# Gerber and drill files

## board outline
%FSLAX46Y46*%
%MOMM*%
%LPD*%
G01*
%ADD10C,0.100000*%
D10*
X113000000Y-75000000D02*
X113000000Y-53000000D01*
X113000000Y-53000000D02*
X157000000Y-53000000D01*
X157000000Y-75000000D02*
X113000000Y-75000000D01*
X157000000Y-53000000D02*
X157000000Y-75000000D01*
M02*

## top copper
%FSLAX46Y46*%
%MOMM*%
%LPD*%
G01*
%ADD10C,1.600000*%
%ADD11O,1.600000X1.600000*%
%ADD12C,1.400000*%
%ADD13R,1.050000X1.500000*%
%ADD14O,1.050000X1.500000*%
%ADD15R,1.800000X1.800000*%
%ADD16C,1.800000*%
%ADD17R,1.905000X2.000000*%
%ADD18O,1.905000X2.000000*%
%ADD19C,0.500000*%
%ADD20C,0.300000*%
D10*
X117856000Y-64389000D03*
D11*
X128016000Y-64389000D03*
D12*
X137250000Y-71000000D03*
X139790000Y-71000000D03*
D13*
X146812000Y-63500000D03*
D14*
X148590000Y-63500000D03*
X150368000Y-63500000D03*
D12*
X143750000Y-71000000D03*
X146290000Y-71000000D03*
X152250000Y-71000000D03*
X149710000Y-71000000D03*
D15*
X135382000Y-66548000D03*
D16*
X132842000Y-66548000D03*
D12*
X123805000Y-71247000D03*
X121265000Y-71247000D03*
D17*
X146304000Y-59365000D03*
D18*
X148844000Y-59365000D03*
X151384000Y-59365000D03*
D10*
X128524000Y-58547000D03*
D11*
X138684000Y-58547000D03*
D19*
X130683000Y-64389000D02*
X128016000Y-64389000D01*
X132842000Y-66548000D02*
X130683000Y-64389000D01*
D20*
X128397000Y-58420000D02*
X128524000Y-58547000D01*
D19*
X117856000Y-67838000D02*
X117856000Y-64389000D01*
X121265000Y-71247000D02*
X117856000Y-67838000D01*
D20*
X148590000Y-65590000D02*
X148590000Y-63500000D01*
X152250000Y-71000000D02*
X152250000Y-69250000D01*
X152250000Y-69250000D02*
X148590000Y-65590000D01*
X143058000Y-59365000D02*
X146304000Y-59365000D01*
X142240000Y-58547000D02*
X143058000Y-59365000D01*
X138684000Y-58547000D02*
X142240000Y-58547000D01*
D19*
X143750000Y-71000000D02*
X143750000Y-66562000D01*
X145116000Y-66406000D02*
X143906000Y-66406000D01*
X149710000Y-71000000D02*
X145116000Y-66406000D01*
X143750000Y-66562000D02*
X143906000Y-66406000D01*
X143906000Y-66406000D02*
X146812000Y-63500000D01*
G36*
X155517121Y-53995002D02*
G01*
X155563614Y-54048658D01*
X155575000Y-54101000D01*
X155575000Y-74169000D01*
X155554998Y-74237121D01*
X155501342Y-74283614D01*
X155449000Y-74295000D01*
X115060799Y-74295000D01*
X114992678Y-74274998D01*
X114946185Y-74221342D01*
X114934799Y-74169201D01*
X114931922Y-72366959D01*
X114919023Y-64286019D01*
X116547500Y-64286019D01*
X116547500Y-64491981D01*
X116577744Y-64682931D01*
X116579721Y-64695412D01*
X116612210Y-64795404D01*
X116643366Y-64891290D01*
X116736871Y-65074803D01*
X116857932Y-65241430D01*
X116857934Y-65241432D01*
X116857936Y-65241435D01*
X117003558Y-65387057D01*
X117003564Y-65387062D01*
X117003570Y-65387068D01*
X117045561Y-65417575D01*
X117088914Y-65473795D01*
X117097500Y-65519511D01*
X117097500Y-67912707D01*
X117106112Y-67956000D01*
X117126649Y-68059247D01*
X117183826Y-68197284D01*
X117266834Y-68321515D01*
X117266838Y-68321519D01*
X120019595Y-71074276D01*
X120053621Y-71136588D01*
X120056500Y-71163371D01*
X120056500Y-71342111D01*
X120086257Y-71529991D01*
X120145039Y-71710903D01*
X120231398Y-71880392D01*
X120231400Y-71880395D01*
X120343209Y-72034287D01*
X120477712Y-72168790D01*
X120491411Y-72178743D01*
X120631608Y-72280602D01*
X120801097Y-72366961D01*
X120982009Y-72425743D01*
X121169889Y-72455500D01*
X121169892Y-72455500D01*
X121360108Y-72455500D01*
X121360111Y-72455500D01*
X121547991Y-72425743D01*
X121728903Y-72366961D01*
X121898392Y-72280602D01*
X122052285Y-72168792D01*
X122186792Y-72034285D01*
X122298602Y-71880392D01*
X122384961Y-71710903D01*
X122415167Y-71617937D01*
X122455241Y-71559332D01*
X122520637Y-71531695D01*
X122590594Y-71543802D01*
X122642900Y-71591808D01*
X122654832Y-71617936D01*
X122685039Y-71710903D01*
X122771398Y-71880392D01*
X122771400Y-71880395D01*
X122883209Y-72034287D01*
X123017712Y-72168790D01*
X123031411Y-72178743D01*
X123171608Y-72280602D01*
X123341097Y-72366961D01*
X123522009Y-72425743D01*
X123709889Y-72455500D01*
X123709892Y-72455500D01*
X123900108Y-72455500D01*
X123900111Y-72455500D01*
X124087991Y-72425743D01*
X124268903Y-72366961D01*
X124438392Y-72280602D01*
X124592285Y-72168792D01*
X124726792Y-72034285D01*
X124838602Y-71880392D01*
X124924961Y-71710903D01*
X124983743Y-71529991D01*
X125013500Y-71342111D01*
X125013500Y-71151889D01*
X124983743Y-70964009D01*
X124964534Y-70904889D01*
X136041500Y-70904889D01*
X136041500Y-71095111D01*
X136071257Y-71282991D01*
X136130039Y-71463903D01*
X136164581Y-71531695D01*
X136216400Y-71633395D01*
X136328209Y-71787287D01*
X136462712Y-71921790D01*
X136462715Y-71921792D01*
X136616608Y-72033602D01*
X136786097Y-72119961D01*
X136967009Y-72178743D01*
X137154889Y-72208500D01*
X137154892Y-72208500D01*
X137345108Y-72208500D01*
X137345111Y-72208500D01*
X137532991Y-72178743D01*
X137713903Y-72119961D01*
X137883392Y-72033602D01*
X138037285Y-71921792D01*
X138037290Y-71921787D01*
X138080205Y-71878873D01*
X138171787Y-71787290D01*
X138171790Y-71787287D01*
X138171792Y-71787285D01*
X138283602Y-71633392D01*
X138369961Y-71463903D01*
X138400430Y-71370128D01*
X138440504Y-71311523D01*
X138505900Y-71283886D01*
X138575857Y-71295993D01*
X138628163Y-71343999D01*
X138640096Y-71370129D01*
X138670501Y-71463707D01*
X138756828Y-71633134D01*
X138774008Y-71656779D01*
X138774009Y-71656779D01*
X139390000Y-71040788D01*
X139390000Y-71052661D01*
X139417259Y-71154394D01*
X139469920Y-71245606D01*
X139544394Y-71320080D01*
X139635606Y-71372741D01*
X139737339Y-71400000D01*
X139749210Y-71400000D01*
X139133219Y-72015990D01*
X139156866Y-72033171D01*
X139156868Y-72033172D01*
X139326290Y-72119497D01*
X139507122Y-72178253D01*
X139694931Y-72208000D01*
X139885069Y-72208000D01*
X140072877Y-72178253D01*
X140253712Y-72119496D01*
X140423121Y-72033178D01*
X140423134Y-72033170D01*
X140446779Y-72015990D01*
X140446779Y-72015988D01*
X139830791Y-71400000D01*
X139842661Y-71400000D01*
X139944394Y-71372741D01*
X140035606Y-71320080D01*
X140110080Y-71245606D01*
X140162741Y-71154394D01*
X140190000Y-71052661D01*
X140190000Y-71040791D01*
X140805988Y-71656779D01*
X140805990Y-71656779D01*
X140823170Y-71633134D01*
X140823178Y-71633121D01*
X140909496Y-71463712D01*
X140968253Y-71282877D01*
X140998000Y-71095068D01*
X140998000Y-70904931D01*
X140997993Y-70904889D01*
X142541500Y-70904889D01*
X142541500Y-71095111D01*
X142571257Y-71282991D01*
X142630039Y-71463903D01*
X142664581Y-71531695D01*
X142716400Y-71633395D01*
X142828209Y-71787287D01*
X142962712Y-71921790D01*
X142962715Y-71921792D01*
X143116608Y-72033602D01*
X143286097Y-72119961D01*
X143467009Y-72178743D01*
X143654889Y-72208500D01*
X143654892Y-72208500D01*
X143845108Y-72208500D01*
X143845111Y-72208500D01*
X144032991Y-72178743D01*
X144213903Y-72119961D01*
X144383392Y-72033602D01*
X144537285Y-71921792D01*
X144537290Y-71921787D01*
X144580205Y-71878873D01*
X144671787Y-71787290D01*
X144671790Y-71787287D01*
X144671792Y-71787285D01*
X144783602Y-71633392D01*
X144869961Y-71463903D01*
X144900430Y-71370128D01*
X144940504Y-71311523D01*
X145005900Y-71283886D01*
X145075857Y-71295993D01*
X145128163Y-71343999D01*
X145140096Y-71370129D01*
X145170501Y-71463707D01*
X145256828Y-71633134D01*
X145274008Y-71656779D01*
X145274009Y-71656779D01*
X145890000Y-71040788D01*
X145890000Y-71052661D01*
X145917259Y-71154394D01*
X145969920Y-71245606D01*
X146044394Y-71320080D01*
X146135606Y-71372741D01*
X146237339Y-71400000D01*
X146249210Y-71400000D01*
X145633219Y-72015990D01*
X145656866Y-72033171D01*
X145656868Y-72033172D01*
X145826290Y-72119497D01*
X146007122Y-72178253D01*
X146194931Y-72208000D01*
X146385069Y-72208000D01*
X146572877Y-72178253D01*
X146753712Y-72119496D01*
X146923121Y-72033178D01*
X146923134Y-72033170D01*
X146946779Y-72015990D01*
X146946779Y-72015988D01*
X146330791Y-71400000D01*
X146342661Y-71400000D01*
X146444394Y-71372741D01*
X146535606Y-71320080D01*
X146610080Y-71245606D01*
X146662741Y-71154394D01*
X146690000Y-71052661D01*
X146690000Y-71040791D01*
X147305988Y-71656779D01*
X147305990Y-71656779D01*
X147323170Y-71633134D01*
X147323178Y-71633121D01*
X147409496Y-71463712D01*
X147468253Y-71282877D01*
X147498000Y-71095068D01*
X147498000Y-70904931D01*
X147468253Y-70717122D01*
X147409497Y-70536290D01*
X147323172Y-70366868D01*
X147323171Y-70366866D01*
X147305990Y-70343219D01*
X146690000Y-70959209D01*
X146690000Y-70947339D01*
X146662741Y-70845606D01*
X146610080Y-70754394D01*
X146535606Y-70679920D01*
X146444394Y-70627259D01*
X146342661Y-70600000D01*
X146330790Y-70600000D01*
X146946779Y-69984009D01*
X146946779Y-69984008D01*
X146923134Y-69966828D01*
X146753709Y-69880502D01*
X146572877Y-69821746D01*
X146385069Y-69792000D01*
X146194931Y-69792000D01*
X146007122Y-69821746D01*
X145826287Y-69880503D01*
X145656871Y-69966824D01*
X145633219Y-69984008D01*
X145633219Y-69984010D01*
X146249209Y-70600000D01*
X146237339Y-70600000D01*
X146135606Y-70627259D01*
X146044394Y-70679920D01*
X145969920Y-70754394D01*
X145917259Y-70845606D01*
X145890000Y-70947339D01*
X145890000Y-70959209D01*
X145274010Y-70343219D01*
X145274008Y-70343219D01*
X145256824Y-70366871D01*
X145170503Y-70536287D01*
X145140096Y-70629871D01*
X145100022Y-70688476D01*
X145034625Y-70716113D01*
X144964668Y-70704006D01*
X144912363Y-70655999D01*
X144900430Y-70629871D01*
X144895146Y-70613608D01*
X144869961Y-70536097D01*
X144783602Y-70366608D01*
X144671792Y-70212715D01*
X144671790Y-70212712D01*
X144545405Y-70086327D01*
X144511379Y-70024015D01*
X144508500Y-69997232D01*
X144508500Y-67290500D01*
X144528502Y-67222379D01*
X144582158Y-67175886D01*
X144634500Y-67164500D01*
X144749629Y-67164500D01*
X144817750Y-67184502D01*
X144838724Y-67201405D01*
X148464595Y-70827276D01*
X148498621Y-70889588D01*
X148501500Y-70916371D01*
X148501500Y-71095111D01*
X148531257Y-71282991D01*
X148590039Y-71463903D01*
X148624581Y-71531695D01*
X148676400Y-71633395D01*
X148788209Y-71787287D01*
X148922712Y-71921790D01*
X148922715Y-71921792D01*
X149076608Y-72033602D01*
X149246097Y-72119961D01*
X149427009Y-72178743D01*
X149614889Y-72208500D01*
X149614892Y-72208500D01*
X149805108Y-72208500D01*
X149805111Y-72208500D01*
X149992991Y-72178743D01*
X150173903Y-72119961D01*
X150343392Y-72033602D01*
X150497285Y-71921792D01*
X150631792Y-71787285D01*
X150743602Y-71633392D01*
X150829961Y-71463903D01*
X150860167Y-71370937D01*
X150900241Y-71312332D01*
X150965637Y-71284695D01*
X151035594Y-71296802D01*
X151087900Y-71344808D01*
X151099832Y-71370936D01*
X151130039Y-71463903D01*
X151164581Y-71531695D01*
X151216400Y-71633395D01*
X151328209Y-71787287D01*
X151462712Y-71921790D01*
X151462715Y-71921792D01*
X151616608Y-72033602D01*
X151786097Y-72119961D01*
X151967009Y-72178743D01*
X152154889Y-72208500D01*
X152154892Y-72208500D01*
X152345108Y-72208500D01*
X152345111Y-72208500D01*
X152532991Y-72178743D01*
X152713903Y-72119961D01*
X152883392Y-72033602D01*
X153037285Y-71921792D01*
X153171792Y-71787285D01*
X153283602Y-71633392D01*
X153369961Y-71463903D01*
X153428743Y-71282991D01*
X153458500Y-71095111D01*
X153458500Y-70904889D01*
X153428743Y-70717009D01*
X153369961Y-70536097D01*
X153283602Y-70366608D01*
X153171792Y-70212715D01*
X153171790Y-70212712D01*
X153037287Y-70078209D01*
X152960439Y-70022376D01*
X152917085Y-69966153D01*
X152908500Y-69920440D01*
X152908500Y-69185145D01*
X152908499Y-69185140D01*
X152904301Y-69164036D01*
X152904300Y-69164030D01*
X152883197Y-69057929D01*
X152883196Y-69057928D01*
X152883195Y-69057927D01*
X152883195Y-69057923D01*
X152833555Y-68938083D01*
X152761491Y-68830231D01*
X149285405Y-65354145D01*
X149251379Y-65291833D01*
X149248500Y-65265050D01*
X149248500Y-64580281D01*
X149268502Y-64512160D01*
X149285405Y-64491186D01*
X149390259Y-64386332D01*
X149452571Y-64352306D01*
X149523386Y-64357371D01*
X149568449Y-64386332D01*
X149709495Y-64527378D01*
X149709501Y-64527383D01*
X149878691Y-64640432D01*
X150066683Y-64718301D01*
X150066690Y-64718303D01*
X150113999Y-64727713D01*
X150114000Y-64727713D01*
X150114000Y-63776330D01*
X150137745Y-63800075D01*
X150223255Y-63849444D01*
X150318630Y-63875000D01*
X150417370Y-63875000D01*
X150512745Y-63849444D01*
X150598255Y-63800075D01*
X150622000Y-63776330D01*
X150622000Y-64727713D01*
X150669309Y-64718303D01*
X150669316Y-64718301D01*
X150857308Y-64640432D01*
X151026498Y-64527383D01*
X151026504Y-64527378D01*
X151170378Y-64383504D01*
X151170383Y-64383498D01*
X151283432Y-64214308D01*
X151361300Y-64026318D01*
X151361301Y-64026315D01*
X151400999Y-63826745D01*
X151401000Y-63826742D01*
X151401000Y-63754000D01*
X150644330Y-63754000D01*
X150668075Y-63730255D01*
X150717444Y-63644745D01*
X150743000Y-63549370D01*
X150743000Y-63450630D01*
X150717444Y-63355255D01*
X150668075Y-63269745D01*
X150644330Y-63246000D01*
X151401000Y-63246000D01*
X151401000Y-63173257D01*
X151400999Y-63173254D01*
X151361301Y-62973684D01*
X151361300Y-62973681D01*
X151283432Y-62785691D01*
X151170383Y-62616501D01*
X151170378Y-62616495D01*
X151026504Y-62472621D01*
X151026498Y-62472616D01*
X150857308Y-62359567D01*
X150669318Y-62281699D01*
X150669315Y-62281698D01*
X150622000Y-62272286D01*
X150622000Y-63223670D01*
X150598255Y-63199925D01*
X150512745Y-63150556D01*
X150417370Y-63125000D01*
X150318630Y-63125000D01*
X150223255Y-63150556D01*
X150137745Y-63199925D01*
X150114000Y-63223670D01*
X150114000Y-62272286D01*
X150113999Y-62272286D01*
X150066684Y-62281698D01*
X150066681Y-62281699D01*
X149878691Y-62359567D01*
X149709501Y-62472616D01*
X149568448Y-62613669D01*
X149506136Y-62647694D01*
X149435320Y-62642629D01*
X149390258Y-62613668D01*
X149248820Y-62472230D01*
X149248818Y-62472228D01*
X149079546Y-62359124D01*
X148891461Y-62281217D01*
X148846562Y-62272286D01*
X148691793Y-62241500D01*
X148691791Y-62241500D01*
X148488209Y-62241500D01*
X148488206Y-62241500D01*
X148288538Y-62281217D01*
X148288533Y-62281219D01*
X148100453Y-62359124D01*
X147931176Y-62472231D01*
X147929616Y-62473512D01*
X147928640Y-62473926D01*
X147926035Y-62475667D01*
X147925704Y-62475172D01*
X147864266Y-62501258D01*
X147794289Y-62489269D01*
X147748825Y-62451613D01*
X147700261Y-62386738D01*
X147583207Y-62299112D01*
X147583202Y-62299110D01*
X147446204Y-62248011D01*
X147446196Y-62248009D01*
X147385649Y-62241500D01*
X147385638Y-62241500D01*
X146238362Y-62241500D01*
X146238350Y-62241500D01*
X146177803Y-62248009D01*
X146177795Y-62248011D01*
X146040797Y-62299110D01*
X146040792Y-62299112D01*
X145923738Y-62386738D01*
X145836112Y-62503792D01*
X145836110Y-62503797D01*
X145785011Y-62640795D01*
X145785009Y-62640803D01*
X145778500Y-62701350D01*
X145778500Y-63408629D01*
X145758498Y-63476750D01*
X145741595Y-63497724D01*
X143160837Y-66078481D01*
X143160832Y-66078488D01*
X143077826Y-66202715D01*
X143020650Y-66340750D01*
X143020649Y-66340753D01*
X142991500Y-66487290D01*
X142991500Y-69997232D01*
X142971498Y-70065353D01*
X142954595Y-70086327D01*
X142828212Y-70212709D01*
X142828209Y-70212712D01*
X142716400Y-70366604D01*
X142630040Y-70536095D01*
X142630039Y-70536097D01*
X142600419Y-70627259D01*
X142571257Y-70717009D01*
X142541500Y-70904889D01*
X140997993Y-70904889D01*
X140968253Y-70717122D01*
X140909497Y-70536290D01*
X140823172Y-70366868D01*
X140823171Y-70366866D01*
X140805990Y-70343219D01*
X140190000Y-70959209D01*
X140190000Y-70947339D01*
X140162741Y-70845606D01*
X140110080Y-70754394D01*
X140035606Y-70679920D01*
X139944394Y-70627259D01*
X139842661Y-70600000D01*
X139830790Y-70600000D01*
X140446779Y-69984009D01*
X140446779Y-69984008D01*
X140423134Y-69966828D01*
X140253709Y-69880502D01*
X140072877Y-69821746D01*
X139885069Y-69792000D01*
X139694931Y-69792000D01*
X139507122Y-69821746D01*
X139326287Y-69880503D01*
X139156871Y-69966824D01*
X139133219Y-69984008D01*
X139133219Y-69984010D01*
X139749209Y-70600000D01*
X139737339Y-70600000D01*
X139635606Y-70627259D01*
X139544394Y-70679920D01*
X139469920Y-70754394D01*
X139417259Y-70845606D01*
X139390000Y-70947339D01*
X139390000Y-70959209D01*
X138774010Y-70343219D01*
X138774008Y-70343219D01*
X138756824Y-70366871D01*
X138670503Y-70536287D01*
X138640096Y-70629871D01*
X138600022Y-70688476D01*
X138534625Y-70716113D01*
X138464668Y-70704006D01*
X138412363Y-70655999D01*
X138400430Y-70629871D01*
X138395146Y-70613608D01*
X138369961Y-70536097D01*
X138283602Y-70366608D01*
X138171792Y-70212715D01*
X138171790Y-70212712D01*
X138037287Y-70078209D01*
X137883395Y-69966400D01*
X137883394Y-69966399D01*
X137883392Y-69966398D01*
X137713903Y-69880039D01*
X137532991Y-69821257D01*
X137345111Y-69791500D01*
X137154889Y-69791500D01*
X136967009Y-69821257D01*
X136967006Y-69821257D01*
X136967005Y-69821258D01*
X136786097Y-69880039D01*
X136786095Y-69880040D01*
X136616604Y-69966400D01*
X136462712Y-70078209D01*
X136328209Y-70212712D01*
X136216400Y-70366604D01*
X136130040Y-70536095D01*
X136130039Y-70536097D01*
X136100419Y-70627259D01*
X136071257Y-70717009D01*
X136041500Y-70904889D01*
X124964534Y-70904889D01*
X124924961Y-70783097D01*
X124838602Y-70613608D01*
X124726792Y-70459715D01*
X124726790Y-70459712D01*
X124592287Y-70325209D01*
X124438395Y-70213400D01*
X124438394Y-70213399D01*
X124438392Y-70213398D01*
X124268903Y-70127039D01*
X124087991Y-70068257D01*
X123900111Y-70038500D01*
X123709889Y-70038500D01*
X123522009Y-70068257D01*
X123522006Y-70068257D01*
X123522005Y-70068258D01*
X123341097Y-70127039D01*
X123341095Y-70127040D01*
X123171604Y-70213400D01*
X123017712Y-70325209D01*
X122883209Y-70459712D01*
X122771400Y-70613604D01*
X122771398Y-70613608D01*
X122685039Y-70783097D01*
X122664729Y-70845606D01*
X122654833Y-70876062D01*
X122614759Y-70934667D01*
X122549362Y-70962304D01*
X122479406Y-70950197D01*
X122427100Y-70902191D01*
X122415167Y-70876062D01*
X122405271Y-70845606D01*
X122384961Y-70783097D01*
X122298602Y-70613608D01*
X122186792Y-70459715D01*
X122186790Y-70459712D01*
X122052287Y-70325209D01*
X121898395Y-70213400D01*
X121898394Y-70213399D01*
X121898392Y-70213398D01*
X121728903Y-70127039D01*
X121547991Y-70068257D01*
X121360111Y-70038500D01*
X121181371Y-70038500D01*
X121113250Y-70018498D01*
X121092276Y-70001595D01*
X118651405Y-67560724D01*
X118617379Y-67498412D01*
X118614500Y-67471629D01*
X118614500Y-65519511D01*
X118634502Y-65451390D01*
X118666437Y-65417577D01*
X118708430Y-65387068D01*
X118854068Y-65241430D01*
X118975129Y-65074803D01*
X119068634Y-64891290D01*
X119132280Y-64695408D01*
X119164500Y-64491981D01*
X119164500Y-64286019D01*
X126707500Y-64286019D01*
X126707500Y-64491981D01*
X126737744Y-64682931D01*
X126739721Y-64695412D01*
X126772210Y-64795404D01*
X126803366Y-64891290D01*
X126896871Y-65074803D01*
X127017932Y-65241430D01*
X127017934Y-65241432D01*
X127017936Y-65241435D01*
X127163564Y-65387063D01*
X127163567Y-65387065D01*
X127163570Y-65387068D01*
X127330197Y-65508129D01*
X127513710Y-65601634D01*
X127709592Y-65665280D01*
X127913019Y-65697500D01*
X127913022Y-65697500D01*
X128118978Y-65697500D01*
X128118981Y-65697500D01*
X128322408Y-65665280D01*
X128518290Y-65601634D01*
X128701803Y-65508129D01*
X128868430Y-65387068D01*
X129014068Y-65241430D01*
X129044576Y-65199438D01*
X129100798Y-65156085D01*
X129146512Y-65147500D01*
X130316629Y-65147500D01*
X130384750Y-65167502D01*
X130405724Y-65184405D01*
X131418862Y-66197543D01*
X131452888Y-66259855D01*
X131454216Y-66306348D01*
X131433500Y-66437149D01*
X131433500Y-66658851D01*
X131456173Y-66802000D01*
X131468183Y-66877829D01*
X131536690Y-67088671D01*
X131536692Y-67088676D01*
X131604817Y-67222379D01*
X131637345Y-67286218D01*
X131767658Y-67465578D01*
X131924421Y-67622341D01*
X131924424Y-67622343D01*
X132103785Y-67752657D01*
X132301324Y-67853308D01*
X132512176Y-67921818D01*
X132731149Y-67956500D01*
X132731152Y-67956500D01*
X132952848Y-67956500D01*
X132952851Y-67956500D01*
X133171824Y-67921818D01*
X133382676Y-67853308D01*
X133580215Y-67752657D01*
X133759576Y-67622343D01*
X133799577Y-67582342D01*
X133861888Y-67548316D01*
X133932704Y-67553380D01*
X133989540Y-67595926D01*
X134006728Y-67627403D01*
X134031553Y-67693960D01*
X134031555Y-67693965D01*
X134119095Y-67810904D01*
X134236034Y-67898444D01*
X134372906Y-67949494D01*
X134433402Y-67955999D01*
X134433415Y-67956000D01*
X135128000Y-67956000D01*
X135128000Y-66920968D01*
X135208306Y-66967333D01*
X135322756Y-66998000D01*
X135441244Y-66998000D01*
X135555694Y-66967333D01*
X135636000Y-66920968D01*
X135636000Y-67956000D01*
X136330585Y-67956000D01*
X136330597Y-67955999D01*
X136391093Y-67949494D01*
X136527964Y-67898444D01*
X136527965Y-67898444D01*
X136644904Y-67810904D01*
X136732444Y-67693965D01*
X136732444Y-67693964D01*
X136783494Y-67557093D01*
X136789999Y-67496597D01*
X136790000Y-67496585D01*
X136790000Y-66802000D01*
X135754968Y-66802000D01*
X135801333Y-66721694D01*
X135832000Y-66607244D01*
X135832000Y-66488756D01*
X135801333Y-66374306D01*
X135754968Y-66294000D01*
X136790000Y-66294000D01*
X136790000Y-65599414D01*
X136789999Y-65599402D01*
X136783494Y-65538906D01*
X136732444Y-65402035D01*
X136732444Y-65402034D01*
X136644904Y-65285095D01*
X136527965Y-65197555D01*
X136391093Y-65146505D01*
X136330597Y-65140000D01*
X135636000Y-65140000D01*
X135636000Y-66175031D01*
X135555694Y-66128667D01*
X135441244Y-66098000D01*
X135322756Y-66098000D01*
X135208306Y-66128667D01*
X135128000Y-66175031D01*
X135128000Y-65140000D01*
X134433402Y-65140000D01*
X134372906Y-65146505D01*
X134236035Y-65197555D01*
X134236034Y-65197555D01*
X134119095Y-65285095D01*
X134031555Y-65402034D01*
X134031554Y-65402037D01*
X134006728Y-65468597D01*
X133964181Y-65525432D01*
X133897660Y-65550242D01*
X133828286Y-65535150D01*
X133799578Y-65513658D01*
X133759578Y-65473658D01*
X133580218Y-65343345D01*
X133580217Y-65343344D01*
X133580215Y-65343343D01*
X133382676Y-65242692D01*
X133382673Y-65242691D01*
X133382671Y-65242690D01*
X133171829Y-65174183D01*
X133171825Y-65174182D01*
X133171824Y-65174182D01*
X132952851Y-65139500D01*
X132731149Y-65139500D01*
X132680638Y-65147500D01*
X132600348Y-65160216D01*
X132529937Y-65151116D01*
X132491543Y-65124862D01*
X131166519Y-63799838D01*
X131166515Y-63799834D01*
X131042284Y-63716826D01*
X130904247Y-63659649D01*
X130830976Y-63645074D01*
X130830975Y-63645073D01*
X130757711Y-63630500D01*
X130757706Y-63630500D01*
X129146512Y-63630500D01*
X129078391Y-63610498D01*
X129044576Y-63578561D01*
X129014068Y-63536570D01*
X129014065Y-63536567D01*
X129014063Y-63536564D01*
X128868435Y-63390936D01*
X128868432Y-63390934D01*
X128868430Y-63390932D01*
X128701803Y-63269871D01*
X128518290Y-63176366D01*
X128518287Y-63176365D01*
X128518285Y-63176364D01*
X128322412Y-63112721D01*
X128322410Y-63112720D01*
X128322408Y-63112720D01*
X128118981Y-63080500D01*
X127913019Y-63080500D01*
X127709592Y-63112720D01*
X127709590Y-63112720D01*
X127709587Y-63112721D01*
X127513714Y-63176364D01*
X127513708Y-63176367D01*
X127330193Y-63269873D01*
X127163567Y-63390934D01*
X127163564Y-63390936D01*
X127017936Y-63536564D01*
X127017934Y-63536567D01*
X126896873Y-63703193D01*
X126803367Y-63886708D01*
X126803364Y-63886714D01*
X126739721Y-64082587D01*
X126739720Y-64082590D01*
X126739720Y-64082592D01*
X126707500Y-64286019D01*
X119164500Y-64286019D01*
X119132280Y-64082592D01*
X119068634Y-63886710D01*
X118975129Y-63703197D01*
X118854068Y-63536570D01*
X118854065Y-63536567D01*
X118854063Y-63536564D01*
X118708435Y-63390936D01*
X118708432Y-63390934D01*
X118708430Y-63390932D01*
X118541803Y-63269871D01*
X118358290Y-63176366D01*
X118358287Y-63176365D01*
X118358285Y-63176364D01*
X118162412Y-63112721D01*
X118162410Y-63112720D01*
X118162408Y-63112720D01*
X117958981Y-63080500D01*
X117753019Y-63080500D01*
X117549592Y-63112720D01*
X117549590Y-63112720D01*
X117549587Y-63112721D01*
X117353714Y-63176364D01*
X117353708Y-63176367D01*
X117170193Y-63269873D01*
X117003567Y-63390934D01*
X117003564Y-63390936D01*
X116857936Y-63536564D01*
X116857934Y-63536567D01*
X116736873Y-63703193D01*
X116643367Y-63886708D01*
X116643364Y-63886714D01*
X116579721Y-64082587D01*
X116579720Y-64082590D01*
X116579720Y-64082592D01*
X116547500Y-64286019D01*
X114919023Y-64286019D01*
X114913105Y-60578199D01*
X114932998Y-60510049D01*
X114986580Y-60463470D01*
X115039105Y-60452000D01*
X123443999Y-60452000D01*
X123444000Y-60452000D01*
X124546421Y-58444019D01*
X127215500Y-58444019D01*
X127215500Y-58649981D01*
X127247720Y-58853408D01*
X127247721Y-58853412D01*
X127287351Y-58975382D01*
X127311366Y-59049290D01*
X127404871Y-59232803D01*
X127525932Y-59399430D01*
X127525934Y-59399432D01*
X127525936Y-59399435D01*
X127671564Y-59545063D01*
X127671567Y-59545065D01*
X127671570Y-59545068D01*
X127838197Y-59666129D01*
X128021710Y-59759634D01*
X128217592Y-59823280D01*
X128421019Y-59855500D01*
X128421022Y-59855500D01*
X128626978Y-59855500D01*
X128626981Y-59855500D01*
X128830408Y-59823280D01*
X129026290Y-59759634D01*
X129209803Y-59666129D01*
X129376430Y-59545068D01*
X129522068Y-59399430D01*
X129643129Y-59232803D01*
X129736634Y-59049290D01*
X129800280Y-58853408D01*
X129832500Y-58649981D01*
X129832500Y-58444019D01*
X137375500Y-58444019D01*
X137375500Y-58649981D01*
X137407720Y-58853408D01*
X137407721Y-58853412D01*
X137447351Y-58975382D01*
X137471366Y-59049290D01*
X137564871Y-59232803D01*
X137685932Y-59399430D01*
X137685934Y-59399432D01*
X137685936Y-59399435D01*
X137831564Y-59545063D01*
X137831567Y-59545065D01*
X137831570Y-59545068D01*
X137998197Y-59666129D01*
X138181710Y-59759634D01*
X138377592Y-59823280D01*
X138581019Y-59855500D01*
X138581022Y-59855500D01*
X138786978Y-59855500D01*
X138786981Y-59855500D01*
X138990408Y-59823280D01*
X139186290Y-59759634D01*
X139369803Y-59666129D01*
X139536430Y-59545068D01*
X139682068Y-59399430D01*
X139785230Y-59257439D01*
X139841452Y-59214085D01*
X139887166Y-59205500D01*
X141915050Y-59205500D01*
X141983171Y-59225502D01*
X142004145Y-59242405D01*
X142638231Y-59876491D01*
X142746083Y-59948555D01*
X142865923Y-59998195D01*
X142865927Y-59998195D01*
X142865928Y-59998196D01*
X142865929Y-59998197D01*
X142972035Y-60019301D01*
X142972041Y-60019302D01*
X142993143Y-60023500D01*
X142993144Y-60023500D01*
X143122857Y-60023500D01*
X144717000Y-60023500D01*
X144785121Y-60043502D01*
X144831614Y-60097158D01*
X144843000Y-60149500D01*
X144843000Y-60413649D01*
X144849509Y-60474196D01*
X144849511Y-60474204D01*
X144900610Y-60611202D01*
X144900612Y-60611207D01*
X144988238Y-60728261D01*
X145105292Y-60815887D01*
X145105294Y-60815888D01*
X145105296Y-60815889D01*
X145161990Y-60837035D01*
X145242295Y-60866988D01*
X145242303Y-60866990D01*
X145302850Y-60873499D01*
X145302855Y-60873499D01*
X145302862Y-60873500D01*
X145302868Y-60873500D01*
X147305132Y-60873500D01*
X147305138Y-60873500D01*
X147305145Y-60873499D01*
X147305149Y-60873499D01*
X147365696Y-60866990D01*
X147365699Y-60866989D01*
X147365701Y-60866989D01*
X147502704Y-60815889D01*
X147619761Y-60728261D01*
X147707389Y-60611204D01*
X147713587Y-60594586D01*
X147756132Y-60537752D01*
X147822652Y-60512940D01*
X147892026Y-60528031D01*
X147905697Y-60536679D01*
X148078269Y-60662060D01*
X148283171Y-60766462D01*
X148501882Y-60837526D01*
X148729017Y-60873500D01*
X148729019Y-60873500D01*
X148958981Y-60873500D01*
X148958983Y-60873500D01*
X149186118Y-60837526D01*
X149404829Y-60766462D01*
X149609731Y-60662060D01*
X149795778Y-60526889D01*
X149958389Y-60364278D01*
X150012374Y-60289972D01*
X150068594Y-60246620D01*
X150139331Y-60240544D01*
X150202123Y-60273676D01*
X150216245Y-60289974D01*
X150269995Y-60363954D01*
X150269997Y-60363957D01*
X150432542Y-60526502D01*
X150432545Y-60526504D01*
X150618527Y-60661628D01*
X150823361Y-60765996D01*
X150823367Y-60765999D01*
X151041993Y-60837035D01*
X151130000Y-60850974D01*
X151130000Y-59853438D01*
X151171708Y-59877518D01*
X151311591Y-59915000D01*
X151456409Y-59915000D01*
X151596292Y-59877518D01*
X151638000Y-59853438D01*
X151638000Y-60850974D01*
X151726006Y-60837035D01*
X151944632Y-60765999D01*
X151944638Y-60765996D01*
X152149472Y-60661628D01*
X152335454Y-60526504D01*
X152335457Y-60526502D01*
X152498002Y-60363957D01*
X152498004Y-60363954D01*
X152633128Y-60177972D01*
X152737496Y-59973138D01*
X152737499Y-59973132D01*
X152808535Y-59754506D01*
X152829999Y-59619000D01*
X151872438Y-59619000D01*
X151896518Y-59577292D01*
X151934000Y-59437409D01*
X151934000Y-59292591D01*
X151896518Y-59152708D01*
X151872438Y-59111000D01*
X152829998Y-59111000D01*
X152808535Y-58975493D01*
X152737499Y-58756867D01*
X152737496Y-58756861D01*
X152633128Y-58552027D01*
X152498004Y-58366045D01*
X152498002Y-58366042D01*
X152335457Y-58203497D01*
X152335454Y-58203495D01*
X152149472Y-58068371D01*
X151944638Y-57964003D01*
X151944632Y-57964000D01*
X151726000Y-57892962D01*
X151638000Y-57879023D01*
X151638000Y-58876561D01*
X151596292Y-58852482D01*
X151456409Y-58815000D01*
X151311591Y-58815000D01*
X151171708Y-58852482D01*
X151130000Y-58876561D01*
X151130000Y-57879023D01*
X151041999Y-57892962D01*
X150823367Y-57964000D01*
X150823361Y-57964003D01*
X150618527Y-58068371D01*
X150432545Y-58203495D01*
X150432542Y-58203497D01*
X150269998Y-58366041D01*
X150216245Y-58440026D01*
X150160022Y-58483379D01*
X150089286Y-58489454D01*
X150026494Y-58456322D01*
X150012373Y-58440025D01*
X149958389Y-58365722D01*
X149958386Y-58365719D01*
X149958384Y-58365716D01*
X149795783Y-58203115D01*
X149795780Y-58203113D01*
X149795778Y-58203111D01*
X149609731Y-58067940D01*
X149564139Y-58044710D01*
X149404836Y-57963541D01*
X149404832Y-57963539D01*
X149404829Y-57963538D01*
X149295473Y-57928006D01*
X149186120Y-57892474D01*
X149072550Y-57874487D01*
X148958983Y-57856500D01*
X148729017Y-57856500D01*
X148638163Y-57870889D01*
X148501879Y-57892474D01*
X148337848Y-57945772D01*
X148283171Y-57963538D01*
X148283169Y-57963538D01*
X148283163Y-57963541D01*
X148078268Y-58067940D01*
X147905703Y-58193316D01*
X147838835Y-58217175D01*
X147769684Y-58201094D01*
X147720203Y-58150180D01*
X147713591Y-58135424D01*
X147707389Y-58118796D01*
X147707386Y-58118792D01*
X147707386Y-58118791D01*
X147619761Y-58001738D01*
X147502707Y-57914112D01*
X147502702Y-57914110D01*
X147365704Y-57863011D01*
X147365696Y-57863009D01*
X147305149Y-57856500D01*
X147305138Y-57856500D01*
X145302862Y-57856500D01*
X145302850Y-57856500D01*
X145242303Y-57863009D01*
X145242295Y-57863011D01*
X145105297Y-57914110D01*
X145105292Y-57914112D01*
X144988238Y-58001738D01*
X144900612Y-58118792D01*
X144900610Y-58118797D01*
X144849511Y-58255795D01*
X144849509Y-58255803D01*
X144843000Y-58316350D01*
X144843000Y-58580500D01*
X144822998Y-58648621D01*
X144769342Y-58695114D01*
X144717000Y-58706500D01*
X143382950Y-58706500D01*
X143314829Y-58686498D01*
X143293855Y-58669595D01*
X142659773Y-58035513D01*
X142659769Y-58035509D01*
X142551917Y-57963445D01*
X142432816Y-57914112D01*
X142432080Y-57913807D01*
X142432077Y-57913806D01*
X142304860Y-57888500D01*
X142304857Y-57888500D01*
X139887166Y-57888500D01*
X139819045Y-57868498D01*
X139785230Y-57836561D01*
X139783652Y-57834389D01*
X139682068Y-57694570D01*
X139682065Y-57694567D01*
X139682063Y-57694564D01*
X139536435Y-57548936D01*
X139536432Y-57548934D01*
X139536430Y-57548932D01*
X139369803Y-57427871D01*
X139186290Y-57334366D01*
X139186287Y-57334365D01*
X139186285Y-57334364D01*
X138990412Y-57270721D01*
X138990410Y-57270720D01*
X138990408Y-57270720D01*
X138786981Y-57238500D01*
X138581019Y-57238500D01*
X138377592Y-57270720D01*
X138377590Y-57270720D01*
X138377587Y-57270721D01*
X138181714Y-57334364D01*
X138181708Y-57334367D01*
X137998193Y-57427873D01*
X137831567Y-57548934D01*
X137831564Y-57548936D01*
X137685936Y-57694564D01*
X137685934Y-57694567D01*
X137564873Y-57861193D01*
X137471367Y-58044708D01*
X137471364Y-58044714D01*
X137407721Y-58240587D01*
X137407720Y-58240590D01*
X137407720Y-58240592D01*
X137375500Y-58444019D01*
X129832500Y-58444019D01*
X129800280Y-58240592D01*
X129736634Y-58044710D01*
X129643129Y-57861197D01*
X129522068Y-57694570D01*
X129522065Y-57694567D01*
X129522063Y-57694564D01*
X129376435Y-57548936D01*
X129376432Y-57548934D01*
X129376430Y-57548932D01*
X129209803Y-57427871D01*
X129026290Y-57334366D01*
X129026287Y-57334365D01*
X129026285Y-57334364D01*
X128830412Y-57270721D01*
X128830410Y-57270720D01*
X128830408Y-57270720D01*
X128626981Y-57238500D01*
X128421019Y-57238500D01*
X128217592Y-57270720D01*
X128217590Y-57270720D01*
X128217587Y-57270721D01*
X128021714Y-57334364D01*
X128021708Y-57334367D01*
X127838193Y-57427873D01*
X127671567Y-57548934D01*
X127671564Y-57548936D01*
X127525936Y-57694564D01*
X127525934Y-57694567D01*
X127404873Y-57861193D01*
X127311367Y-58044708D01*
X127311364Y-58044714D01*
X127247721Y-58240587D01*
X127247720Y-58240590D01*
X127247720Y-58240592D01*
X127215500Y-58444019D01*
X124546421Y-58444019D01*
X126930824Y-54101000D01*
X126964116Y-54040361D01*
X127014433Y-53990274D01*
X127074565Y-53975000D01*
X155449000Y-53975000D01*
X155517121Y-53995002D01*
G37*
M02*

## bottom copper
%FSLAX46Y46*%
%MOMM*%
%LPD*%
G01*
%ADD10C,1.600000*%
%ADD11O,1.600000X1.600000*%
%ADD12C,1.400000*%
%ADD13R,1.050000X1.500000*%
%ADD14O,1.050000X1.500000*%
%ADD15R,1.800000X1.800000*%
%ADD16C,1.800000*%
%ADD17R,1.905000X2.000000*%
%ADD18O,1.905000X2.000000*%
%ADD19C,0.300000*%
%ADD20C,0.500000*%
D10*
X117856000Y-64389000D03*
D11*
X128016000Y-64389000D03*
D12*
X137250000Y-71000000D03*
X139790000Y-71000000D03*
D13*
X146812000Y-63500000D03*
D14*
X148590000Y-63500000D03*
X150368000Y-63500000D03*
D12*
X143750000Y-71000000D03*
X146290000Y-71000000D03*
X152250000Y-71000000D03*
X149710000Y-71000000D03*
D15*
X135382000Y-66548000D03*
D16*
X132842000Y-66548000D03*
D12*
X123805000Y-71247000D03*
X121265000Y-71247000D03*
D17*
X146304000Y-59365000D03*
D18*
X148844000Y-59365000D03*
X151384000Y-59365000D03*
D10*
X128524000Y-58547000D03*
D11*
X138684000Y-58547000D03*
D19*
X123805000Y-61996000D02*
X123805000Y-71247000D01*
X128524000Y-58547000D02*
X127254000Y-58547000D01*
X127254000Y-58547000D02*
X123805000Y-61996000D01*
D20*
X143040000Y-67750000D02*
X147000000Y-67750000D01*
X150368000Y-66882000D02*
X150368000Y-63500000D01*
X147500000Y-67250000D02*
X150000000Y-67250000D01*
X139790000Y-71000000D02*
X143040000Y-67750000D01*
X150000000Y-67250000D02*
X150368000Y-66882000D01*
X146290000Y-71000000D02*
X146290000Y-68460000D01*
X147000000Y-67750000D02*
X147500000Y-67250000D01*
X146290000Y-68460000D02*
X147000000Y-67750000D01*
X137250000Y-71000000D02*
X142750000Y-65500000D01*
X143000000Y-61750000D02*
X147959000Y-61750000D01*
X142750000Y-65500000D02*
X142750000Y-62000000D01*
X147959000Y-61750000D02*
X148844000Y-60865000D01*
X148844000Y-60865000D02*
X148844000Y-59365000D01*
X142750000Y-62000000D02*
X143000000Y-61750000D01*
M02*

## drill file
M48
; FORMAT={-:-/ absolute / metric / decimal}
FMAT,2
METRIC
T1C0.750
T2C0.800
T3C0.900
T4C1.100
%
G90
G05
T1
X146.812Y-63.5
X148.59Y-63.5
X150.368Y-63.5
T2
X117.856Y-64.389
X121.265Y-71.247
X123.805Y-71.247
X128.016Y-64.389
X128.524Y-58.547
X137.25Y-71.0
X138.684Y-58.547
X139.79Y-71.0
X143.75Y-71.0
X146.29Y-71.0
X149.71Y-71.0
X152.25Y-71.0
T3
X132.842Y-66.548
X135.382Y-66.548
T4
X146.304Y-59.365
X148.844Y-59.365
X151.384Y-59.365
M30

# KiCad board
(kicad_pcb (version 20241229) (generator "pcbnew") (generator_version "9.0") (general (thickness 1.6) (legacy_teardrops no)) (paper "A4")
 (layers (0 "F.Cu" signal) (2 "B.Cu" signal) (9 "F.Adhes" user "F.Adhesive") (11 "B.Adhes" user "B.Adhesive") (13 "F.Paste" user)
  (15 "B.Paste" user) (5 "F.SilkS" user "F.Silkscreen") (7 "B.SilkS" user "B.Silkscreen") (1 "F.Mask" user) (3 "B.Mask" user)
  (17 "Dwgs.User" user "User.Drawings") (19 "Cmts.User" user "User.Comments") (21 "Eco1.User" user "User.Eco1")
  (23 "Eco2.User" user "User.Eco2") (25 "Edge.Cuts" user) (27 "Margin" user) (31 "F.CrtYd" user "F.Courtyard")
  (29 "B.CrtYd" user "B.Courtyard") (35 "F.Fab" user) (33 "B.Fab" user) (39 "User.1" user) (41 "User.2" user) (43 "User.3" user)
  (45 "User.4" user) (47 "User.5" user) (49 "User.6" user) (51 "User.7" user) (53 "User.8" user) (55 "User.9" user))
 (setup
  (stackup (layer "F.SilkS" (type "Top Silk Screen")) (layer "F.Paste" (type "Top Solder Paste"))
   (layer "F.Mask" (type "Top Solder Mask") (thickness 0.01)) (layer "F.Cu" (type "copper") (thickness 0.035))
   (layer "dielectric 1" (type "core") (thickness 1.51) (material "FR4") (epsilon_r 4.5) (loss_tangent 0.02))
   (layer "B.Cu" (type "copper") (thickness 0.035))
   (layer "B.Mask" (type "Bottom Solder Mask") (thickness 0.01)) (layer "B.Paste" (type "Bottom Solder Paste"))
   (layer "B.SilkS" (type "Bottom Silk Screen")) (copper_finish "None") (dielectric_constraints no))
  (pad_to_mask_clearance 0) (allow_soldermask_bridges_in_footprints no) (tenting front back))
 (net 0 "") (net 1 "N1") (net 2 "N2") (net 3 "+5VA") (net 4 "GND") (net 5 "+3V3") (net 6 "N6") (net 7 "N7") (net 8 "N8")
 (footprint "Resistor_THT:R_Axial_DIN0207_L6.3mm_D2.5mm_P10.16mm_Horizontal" (layer "F.Cu") (at 117.856 64.389)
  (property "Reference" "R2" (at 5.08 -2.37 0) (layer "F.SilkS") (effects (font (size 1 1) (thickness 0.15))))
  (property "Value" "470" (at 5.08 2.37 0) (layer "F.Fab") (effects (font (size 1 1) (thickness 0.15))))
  (pad "1" thru_hole circle (at 0 0) (size 1.6 1.6) (drill 0.8) (layers "*.Cu" "*.Mask") (remove_unused_layers no) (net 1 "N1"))
  (pad "2" thru_hole oval (at 10.16 0) (size 1.6 1.6) (drill 0.8) (layers "*.Cu" "*.Mask") (remove_unused_layers no) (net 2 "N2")))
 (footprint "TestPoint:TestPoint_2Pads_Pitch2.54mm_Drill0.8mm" (layer "F.Cu") (at 137.25 71)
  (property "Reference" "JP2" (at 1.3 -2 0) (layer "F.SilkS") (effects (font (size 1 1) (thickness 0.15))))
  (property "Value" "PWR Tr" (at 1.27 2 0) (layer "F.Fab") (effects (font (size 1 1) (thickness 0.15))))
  (pad "1" thru_hole circle (at 0 0) (size 1.4 1.4) (drill 0.8) (layers "*.Cu" "*.Mask") (remove_unused_layers no) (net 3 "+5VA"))
  (pad "2" thru_hole circle (at 2.54 0) (size 1.4 1.4) (drill 0.8) (layers "*.Cu" "*.Mask") (remove_unused_layers no) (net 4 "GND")))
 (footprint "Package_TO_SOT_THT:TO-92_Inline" (layer "F.Cu") (at 147.32 63.5)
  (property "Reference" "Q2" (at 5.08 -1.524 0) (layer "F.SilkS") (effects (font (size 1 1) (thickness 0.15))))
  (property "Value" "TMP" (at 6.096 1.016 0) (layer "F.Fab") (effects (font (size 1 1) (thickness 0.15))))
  (pad "1" thru_hole rect (at -0.508 0) (size 1.05 1.5) (drill 0.75) (layers "*.Cu" "*.Mask") (remove_unused_layers no) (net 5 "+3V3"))
  (pad "2" thru_hole oval (at 1.27 0) (size 1.05 1.5) (drill 0.75) (layers "*.Cu" "*.Mask") (remove_unused_layers no) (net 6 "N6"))
  (pad "3" thru_hole oval (at 3.048 0) (size 1.05 1.5) (drill 0.75) (layers "*.Cu" "*.Mask") (remove_unused_layers no) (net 4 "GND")))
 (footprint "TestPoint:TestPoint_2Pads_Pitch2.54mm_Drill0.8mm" (layer "F.Cu") (at 143.75 71)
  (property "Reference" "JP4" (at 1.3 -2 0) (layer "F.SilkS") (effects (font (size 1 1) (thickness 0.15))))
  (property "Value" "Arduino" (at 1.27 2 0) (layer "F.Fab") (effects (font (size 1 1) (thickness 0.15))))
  (pad "1" thru_hole circle (at 0 0) (size 1.4 1.4) (drill 0.8) (layers "*.Cu" "*.Mask") (remove_unused_layers no) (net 5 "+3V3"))
  (pad "2" thru_hole circle (at 2.54 0) (size 1.4 1.4) (drill 0.8) (layers "*.Cu" "*.Mask") (remove_unused_layers no) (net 4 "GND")))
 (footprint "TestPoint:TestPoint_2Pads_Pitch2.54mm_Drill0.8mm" (layer "F.Cu") (at 152.25 71 180)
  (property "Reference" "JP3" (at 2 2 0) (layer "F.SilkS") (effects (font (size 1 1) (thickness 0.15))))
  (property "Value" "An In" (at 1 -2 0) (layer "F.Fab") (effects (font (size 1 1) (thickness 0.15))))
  (pad "1" thru_hole circle (at 0 0 180) (size 1.4 1.4) (drill 0.8) (layers "*.Cu" "*.Mask") (remove_unused_layers no) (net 6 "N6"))
  (pad "2" thru_hole circle (at 2.54 0 180) (size 1.4 1.4) (drill 0.8) (layers "*.Cu" "*.Mask") (remove_unused_layers no) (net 5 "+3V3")))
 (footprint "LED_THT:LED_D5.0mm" (layer "F.Cu") (at 135.382 66.548 180)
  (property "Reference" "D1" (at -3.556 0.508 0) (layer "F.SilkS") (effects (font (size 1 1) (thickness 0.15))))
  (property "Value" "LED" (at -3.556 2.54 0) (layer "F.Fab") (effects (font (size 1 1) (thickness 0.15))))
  (pad "1" thru_hole rect (at 0 0 180) (size 1.8 1.8) (drill 0.9) (layers "*.Cu" "*.Mask") (remove_unused_layers no) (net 4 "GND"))
  (pad "2" thru_hole circle (at 2.54 0 180) (size 1.8 1.8) (drill 0.9) (layers "*.Cu" "*.Mask") (remove_unused_layers no) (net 2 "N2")))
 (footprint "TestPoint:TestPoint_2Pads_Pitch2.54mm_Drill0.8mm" (layer "F.Cu") (at 123.805 71.247 180)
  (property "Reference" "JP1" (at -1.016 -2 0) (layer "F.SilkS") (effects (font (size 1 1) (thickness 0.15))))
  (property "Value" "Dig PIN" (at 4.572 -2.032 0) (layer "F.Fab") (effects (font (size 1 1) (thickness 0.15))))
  (pad "1" thru_hole circle (at 0 0 180) (size 1.4 1.4) (drill 0.8) (layers "*.Cu" "*.Mask") (remove_unused_layers no) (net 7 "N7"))
  (pad "2" thru_hole circle (at 2.54 0 180) (size 1.4 1.4) (drill 0.8) (layers "*.Cu" "*.Mask") (remove_unused_layers no) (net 1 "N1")))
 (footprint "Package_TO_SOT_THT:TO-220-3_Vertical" (layer "F.Cu") (at 146.304 59.365)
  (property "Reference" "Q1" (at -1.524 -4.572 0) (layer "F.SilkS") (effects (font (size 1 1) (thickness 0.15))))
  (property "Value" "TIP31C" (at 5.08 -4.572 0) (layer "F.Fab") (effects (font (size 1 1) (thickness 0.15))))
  (pad "1" thru_hole rect (at 0 0) (size 1.905 2) (drill 1.1) (layers "*.Cu" "*.Mask") (remove_unused_layers no) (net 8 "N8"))
  (pad "2" thru_hole oval (at 2.54 0) (size 1.905 2) (drill 1.1) (layers "*.Cu" "*.Mask") (remove_unused_layers no) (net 3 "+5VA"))
  (pad "3" thru_hole oval (at 5.08 0) (size 1.905 2) (drill 1.1) (layers "*.Cu" "*.Mask") (remove_unused_layers no) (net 4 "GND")))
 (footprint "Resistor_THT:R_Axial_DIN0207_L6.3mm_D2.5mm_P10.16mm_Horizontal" (layer "F.Cu") (at 128.524 58.547)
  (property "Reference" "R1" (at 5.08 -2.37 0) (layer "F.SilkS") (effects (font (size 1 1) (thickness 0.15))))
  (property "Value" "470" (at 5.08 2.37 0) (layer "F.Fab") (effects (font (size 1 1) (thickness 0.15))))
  (pad "1" thru_hole circle (at 0 0) (size 1.6 1.6) (drill 0.8) (layers "*.Cu" "*.Mask") (remove_unused_layers no) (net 7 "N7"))
  (pad "2" thru_hole oval (at 10.16 0) (size 1.6 1.6) (drill 0.8) (layers "*.Cu" "*.Mask") (remove_unused_layers no) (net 8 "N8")))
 (gr_line (start 113 75) (end 113 53) (stroke (width 0.1) (type solid)) (layer "Edge.Cuts"))
 (gr_line (start 113 53) (end 157 53) (stroke (width 0.1) (type solid)) (layer "Edge.Cuts"))
 (gr_line (start 157 75) (end 113 75) (stroke (width 0.1) (type solid)) (layer "Edge.Cuts"))
 (gr_line (start 157 53) (end 157 75) (stroke (width 0.1) (type solid)) (layer "Edge.Cuts"))
 (segment (start 130.683 64.389) (end 128.016 64.389) (width 0.5) (layer "F.Cu") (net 2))
 (segment (start 132.842 66.548) (end 130.683 64.389) (width 0.5) (layer "F.Cu") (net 2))
 (segment (start 128.397 58.42) (end 128.524 58.547) (width 0.3) (layer "F.Cu") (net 7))
 (segment (start 123.805 61.996) (end 123.805 71.247) (width 0.3) (layer "B.Cu") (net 7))
 (segment (start 128.524 58.547) (end 127.254 58.547) (width 0.3) (layer "B.Cu") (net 7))
 (segment (start 127.254 58.547) (end 123.805 61.996) (width 0.3) (layer "B.Cu") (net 7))
 (segment (start 117.856 67.838) (end 117.856 64.389) (width 0.5) (layer "F.Cu") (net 1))
 (segment (start 121.265 71.247) (end 117.856 67.838) (width 0.5) (layer "F.Cu") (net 1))
 (segment (start 148.59 65.59) (end 148.59 63.5) (width 0.3) (layer "F.Cu") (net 6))
 (segment (start 152.25 71) (end 152.25 69.25) (width 0.3) (layer "F.Cu") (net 6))
 (segment (start 152.25 69.25) (end 148.59 65.59) (width 0.3) (layer "F.Cu") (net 6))
 (segment (start 143.058 59.365) (end 146.304 59.365) (width 0.3) (layer "F.Cu") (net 8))
 (segment (start 142.24 58.547) (end 143.058 59.365) (width 0.3) (layer "F.Cu") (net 8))
 (segment (start 138.684 58.547) (end 142.24 58.547) (width 0.3) (layer "F.Cu") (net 8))
 (segment (start 143.04 67.75) (end 147 67.75) (width 0.5) (layer "B.Cu") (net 4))
 (segment (start 150.368 66.882) (end 150.368 63.5) (width 0.5) (layer "B.Cu") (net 4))
 (segment (start 147.5 67.25) (end 150 67.25) (width 0.5) (layer "B.Cu") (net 4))
 (segment (start 139.79 71) (end 143.04 67.75) (width 0.5) (layer "B.Cu") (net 4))
 (segment (start 150 67.25) (end 150.368 66.882) (width 0.5) (layer "B.Cu") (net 4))
 (segment (start 146.29 71) (end 146.29 68.46) (width 0.5) (layer "B.Cu") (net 4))
 (segment (start 147 67.75) (end 147.5 67.25) (width 0.5) (layer "B.Cu") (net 4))
 (segment (start 146.29 68.46) (end 147 67.75) (width 0.5) (layer "B.Cu") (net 4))
 (segment (start 137.25 71) (end 142.75 65.5) (width 0.5) (layer "B.Cu") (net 3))
 (segment (start 143 61.75) (end 147.959 61.75) (width 0.5) (layer "B.Cu") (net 3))
 (segment (start 142.75 65.5) (end 142.75 62) (width 0.5) (layer "B.Cu") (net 3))
 (segment (start 147.959 61.75) (end 148.844 60.865) (width 0.5) (layer "B.Cu") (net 3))
 (segment (start 148.844 60.865) (end 148.844 59.365) (width 0.5) (layer "B.Cu") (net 3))
 (segment (start 142.75 62) (end 143 61.75) (width 0.5) (layer "B.Cu") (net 3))
 (segment (start 143.75 71) (end 143.75 66.562) (width 0.5) (layer "F.Cu") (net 5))
 (segment (start 145.116 66.406) (end 143.906 66.406) (width 0.5) (layer "F.Cu") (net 5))
 (segment (start 149.71 71) (end 145.116 66.406) (width 0.5) (layer "F.Cu") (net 5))
 (segment (start 143.75 66.562) (end 143.906 66.406) (width 0.5) (layer "F.Cu") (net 5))
 (segment (start 143.906 66.406) (end 146.812 63.5) (width 0.5) (layer "F.Cu") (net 5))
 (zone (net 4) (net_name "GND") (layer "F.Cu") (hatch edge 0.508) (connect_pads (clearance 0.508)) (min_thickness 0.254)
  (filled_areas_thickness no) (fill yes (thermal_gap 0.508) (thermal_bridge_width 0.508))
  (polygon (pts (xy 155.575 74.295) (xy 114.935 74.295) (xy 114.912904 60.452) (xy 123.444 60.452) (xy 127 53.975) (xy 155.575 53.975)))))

